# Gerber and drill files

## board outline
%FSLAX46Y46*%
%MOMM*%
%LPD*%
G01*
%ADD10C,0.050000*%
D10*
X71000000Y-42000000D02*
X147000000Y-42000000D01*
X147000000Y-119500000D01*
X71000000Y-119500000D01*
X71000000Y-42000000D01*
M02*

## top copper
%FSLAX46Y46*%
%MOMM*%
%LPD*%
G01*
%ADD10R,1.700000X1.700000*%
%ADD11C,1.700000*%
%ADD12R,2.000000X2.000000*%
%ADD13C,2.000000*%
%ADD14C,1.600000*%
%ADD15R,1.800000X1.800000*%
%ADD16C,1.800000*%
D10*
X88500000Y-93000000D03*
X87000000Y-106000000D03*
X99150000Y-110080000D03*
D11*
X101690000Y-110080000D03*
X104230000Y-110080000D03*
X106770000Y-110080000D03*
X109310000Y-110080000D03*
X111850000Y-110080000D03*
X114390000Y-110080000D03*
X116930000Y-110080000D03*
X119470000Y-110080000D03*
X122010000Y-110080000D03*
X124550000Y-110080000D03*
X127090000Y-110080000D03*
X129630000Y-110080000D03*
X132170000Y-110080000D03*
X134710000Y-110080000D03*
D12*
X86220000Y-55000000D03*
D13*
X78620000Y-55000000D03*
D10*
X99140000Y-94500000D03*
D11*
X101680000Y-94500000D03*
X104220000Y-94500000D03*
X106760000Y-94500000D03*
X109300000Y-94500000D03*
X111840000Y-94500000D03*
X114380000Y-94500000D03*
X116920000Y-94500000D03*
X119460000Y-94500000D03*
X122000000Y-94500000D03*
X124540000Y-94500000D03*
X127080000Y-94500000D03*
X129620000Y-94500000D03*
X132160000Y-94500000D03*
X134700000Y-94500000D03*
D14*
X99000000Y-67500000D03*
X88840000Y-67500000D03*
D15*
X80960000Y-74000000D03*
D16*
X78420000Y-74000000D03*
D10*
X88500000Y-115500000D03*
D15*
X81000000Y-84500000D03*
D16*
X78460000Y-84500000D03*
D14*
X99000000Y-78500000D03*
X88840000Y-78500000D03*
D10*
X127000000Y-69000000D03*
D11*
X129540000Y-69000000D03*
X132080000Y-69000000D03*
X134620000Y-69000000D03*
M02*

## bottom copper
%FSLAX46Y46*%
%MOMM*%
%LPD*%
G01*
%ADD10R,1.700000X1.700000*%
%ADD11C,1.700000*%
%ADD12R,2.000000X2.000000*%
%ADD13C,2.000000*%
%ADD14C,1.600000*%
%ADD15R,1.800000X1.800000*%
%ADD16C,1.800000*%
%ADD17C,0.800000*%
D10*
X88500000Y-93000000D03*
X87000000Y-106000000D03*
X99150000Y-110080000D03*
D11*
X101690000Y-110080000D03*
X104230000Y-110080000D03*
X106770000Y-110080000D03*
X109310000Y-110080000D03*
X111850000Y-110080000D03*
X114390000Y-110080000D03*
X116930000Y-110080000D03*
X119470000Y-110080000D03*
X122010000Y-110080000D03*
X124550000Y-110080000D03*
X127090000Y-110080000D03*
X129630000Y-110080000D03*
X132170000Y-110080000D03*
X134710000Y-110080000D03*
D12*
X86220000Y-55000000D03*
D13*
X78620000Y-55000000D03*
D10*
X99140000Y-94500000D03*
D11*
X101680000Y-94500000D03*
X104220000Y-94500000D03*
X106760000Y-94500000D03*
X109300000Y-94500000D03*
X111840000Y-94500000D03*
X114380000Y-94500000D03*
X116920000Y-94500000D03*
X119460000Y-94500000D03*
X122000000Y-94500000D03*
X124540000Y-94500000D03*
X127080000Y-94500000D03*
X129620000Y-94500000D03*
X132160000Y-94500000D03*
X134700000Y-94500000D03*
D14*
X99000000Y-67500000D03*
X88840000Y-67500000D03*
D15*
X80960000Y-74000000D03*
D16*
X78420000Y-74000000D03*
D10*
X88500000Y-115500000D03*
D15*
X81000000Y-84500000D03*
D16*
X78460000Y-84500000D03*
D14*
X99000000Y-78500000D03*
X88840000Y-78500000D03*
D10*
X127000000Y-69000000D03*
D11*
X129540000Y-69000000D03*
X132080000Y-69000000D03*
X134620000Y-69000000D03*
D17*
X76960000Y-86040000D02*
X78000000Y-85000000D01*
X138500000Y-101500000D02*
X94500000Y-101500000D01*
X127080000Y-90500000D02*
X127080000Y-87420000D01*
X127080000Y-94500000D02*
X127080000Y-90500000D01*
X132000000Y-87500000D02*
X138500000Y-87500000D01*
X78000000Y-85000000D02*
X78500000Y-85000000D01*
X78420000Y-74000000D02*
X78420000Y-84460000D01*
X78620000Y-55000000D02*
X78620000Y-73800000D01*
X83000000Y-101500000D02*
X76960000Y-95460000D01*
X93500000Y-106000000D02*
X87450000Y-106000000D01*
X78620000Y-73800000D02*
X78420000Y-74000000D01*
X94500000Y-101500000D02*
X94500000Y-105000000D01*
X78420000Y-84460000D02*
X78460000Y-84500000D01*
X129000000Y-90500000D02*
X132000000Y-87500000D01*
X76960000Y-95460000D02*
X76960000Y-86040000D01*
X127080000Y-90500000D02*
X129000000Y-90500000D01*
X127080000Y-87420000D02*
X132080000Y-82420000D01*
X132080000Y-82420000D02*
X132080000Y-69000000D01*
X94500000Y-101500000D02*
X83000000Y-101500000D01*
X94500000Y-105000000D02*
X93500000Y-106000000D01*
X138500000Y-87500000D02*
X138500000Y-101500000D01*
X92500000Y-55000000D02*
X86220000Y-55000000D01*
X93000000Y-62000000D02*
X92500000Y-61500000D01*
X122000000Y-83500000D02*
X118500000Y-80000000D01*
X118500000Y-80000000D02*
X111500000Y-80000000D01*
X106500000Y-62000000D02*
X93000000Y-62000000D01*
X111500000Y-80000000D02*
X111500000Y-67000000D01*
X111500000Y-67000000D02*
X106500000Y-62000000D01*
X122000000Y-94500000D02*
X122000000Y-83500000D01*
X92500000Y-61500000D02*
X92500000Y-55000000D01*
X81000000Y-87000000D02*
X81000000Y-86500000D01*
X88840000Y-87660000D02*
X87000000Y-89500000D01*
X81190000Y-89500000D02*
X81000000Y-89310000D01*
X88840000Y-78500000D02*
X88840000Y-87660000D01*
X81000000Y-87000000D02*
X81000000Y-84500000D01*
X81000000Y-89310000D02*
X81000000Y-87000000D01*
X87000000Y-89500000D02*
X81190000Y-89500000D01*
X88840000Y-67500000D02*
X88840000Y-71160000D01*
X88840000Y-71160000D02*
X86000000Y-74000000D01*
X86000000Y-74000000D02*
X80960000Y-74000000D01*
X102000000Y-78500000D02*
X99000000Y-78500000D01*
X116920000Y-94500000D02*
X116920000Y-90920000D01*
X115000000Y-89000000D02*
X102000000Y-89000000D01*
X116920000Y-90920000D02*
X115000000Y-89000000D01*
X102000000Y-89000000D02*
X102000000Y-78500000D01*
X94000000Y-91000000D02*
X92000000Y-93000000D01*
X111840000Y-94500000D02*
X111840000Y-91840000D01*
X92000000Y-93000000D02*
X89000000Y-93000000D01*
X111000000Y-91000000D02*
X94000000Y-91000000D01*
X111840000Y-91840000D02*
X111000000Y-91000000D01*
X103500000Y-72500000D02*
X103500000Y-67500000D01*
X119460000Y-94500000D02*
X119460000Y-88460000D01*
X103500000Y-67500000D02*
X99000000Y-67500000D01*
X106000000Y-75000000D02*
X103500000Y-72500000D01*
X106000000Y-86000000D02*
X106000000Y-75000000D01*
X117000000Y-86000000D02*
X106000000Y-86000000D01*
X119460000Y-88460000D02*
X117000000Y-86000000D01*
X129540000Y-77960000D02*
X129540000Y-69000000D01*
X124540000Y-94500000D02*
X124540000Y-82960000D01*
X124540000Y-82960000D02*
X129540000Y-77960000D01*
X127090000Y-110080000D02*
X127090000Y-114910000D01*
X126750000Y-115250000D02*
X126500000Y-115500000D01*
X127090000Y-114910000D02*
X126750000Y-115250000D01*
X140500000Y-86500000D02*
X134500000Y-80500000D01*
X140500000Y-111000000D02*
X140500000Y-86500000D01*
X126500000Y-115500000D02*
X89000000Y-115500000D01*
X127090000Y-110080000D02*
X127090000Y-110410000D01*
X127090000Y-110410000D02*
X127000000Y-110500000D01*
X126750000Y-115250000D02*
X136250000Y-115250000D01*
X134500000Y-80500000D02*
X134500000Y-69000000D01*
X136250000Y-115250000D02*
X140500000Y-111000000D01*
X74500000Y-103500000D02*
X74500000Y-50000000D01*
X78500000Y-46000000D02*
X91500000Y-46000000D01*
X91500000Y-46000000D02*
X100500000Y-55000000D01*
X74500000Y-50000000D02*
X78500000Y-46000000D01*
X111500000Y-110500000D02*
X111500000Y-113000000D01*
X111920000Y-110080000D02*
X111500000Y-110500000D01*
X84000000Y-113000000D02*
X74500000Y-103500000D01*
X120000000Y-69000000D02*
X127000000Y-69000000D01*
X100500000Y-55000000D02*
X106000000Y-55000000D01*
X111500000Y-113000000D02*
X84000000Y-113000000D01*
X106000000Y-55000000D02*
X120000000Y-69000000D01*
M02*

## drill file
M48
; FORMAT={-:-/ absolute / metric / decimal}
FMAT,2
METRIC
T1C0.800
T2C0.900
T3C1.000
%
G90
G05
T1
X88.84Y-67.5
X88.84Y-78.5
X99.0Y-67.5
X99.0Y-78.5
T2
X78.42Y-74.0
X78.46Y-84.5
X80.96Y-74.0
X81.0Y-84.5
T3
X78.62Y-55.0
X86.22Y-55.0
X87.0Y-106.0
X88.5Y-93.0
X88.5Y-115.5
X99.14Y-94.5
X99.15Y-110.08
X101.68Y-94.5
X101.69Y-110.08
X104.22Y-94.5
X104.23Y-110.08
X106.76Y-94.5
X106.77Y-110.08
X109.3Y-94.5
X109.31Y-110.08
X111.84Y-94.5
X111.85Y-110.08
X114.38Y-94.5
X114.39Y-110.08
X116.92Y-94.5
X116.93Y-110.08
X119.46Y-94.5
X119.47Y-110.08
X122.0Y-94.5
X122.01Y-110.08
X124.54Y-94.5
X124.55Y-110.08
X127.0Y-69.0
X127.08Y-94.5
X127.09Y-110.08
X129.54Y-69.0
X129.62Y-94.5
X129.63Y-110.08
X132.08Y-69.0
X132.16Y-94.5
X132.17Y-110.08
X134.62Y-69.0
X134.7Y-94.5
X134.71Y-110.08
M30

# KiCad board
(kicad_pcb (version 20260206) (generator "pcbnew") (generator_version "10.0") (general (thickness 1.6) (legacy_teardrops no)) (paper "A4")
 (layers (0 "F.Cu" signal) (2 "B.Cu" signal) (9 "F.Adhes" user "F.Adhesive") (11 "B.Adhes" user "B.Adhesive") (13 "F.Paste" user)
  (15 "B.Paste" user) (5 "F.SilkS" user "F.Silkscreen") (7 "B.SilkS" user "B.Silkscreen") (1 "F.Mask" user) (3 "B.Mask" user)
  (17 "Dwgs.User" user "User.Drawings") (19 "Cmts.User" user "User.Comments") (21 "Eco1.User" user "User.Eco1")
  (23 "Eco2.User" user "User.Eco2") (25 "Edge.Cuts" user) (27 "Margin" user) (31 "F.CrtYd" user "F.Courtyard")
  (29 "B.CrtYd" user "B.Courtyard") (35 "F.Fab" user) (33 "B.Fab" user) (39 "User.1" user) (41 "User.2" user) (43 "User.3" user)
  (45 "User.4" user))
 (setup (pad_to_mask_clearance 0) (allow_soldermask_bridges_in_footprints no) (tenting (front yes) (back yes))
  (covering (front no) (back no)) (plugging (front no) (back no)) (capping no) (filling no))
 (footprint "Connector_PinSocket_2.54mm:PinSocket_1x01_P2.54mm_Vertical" (layer "F.Cu") (at 88.5 93 90)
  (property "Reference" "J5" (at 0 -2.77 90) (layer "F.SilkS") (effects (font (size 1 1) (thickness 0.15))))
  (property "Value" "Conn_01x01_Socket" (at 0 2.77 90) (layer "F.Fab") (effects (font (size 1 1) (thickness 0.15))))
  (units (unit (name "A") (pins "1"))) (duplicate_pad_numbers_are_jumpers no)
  (pad "1" thru_hole rect (at 0 0 90) (size 1.7 1.7) (drill 1) (layers "*.Cu" "*.Mask") (remove_unused_layers no) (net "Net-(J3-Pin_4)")))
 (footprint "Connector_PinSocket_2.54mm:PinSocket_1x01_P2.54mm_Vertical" (layer "F.Cu") (at 87 106 90)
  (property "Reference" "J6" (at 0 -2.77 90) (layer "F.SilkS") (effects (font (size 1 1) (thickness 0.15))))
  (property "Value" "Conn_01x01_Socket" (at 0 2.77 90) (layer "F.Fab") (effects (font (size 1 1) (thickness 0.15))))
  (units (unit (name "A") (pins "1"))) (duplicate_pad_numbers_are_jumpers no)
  (pad "1" thru_hole rect (at 0 0 90) (size 1.7 1.7) (drill 1) (layers "*.Cu" "*.Mask") (remove_unused_layers no) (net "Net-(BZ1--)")))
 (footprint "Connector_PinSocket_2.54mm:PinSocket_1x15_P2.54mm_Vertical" (layer "F.Cu") (at 99.15 110.08 90)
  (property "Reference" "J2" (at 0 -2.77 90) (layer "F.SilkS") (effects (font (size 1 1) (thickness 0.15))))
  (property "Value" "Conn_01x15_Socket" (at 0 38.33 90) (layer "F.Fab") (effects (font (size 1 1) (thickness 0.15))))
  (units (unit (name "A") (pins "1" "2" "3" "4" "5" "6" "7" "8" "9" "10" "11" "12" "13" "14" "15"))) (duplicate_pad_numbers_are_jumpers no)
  (pad "1" thru_hole rect (at 0 0 90) (size 1.7 1.7) (drill 1) (layers "*.Cu" "*.Mask") (remove_unused_layers no)
   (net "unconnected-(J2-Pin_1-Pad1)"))
  (pad "2" thru_hole circle (at 0 2.54 90) (size 1.7 1.7) (drill 1) (layers "*.Cu" "*.Mask") (remove_unused_layers no)
   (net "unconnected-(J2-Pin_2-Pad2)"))
  (pad "3" thru_hole circle (at 0 5.08 90) (size 1.7 1.7) (drill 1) (layers "*.Cu" "*.Mask") (remove_unused_layers no)
   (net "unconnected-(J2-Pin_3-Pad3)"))
  (pad "4" thru_hole circle (at 0 7.62 90) (size 1.7 1.7) (drill 1) (layers "*.Cu" "*.Mask") (remove_unused_layers no)
   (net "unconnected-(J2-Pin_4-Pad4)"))
  (pad "5" thru_hole circle (at 0 10.16 90) (size 1.7 1.7) (drill 1) (layers "*.Cu" "*.Mask") (remove_unused_layers no)
   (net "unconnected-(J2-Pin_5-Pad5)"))
  (pad "6" thru_hole circle (at 0 12.7 90) (size 1.7 1.7) (drill 1) (layers "*.Cu" "*.Mask") (remove_unused_layers no)
   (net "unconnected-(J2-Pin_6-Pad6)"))
  (pad "7" thru_hole circle (at 0 15.24 90) (size 1.7 1.7) (drill 1) (layers "*.Cu" "*.Mask") (remove_unused_layers no)
   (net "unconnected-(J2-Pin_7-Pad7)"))
  (pad "8" thru_hole circle (at 0 17.78 90) (size 1.7 1.7) (drill 1) (layers "*.Cu" "*.Mask") (remove_unused_layers no)
   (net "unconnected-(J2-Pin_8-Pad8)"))
  (pad "9" thru_hole circle (at 0 20.32 90) (size 1.7 1.7) (drill 1) (layers "*.Cu" "*.Mask") (remove_unused_layers no)
   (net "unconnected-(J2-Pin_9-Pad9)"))
  (pad "10" thru_hole circle (at 0 22.86 90) (size 1.7 1.7) (drill 1) (layers "*.Cu" "*.Mask") (remove_unused_layers no)
   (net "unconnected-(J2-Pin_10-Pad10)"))
  (pad "11" thru_hole circle (at 0 25.4 90) (size 1.7 1.7) (drill 1) (layers "*.Cu" "*.Mask") (remove_unused_layers no)
   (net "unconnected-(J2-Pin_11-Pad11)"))
  (pad "12" thru_hole circle (at 0 27.94 90) (size 1.7 1.7) (drill 1) (layers "*.Cu" "*.Mask") (remove_unused_layers no)
   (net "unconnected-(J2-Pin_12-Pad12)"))
  (pad "13" thru_hole circle (at 0 30.48 90) (size 1.7 1.7) (drill 1) (layers "*.Cu" "*.Mask") (remove_unused_layers no)
   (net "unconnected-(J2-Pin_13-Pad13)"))
  (pad "14" thru_hole circle (at 0 33.02 90) (size 1.7 1.7) (drill 1) (layers "*.Cu" "*.Mask") (remove_unused_layers no)
   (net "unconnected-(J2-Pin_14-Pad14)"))
  (pad "15" thru_hole circle (at 0 35.56 90) (size 1.7 1.7) (drill 1) (layers "*.Cu" "*.Mask") (remove_unused_layers no)
   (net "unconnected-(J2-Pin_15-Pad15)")))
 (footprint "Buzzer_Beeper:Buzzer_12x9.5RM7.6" (layer "F.Cu") (at 86.22 55 180)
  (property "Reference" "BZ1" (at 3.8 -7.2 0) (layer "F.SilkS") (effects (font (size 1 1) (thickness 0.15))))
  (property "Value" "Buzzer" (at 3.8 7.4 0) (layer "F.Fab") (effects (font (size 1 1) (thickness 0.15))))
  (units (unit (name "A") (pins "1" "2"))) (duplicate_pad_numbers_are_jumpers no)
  (pad "1" thru_hole rect (at 0 0 180) (size 2 2) (drill 1) (layers "*.Cu" "*.Mask") (remove_unused_layers no) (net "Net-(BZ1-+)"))
  (pad "2" thru_hole circle (at 7.6 0 180) (size 2 2) (drill 1) (layers "*.Cu" "*.Mask") (remove_unused_layers no) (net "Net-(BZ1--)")))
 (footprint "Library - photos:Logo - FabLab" (layer "F.Cu") (at 115.5 49)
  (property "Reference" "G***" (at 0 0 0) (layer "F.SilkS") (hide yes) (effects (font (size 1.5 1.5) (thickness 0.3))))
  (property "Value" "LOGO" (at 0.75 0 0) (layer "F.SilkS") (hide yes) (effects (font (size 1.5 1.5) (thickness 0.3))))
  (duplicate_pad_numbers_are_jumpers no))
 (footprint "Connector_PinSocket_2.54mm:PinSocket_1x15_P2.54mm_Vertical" (layer "F.Cu") (at 99.14 94.5 90)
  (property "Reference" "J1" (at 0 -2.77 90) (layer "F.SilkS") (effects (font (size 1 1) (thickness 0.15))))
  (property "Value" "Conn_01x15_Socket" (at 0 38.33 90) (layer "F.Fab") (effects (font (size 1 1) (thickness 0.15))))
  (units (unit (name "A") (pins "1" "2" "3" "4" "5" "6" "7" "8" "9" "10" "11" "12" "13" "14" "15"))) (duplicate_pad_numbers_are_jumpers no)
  (pad "1" thru_hole rect (at 0 0 90) (size 1.7 1.7) (drill 1) (layers "*.Cu" "*.Mask") (remove_unused_layers no)
   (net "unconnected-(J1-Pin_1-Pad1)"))
  (pad "2" thru_hole circle (at 0 2.54 90) (size 1.7 1.7) (drill 1) (layers "*.Cu" "*.Mask") (remove_unused_layers no)
   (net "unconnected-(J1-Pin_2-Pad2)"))
  (pad "3" thru_hole circle (at 0 5.08 90) (size 1.7 1.7) (drill 1) (layers "*.Cu" "*.Mask") (remove_unused_layers no)
   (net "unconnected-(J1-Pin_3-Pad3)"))
  (pad "4" thru_hole circle (at 0 7.62 90) (size 1.7 1.7) (drill 1) (layers "*.Cu" "*.Mask") (remove_unused_layers no)
   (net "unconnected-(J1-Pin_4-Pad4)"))
  (pad "5" thru_hole circle (at 0 10.16 90) (size 1.7 1.7) (drill 1) (layers "*.Cu" "*.Mask") (remove_unused_layers no)
   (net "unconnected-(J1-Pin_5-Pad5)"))
  (pad "6" thru_hole circle (at 0 12.7 90) (size 1.7 1.7) (drill 1) (layers "*.Cu" "*.Mask") (remove_unused_layers no)
   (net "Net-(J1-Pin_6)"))
  (pad "7" thru_hole circle (at 0 15.24 90) (size 1.7 1.7) (drill 1) (layers "*.Cu" "*.Mask") (remove_unused_layers no)
   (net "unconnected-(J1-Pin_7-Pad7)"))
  (pad "8" thru_hole circle (at 0 17.78 90) (size 1.7 1.7) (drill 1) (layers "*.Cu" "*.Mask") (remove_unused_layers no)
   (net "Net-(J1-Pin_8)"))
  (pad "9" thru_hole circle (at 0 20.32 90) (size 1.7 1.7) (drill 1) (layers "*.Cu" "*.Mask") (remove_unused_layers no)
   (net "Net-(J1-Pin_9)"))
  (pad "10" thru_hole circle (at 0 22.86 90) (size 1.7 1.7) (drill 1) (layers "*.Cu" "*.Mask") (remove_unused_layers no) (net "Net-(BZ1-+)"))
  (pad "11" thru_hole circle (at 0 25.4 90) (size 1.7 1.7) (drill 1) (layers "*.Cu" "*.Mask") (remove_unused_layers no)
   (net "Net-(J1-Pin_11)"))
  (pad "12" thru_hole circle (at 0 27.94 90) (size 1.7 1.7) (drill 1) (layers "*.Cu" "*.Mask") (remove_unused_layers no) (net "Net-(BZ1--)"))
  (pad "13" thru_hole circle (at 0 30.48 90) (size 1.7 1.7) (drill 1) (layers "*.Cu" "*.Mask") (remove_unused_layers no)
   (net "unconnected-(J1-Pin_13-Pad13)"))
  (pad "14" thru_hole circle (at 0 33.02 90) (size 1.7 1.7) (drill 1) (layers "*.Cu" "*.Mask") (remove_unused_layers no)
   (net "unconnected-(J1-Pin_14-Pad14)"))
  (pad "15" thru_hole circle (at 0 35.56 90) (size 1.7 1.7) (drill 1) (layers "*.Cu" "*.Mask") (remove_unused_layers no)
   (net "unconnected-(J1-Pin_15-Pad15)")))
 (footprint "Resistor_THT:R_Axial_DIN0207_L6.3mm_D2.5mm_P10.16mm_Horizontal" (layer "F.Cu") (at 99 67.5 180)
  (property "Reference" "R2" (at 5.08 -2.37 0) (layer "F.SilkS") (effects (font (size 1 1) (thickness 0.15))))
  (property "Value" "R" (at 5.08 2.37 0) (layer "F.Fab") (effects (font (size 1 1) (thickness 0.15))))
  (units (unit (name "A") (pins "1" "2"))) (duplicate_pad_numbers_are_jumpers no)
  (pad "1" thru_hole circle (at 0 0 180) (size 1.6 1.6) (drill 0.8) (layers "*.Cu" "*.Mask") (remove_unused_layers no)
   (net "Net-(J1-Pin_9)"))
  (pad "2" thru_hole circle (at 10.16 0 180) (size 1.6 1.6) (drill 0.8) (layers "*.Cu" "*.Mask") (remove_unused_layers no)
   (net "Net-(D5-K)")))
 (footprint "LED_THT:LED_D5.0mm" (layer "F.Cu") (at 80.96 74 180)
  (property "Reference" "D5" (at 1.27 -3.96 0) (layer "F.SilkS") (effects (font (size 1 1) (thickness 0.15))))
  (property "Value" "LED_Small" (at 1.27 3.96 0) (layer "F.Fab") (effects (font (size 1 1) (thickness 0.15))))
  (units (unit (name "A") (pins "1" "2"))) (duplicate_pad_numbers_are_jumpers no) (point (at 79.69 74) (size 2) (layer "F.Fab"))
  (pad "1" thru_hole rect (at 0 0 180) (size 1.8 1.8) (drill 0.9) (layers "*.Cu" "*.Mask") (remove_unused_layers no) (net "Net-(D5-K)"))
  (pad "2" thru_hole circle (at 2.54 0 180) (size 1.8 1.8) (drill 0.9) (layers "*.Cu" "*.Mask") (remove_unused_layers no)
   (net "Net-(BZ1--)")))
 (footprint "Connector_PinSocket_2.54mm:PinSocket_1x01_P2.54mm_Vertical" (layer "F.Cu") (at 88.5 115.5 90)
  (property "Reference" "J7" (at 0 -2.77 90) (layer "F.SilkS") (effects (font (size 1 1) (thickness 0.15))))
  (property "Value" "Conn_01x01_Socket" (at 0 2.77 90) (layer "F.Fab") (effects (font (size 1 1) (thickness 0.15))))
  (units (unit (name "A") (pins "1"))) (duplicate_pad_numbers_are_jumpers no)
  (pad "1" thru_hole rect (at 0 0 90) (size 1.7 1.7) (drill 1) (layers "*.Cu" "*.Mask") (remove_unused_layers no) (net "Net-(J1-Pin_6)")))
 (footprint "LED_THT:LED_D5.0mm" (layer "F.Cu") (at 81 84.5 180)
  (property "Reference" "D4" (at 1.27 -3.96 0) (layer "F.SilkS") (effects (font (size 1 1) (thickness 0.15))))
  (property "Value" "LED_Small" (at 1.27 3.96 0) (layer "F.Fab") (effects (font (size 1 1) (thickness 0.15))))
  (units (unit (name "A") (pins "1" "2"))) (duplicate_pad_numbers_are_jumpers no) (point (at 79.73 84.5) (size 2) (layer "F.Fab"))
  (pad "1" thru_hole rect (at 0 0 180) (size 1.8 1.8) (drill 0.9) (layers "*.Cu" "*.Mask") (remove_unused_layers no) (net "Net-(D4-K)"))
  (pad "2" thru_hole circle (at 2.54 0 180) (size 1.8 1.8) (drill 0.9) (layers "*.Cu" "*.Mask") (remove_unused_layers no)
   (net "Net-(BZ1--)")))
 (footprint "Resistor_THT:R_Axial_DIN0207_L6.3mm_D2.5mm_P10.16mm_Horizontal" (layer "F.Cu") (at 99 78.5 180)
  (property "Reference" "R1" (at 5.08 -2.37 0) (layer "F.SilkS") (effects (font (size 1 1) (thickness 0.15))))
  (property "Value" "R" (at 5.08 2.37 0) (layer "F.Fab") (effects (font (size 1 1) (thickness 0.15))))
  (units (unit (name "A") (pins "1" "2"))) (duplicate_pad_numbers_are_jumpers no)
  (pad "1" thru_hole circle (at 0 0 180) (size 1.6 1.6) (drill 0.8) (layers "*.Cu" "*.Mask") (remove_unused_layers no)
   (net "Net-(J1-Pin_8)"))
  (pad "2" thru_hole circle (at 10.16 0 180) (size 1.6 1.6) (drill 0.8) (layers "*.Cu" "*.Mask") (remove_unused_layers no)
   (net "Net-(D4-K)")))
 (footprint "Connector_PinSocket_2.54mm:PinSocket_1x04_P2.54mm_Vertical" (layer "F.Cu") (at 127 69 90)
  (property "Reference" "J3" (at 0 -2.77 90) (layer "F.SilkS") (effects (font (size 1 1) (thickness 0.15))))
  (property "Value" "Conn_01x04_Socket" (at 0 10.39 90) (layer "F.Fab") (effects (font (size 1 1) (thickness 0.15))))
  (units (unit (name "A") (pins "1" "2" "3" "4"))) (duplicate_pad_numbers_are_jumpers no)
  (pad "1" thru_hole rect (at 0 0 90) (size 1.7 1.7) (drill 1) (layers "*.Cu" "*.Mask") (remove_unused_layers no)
   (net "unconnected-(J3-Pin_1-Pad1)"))
  (pad "2" thru_hole circle (at 0 2.54 90) (size 1.7 1.7) (drill 1) (layers "*.Cu" "*.Mask") (remove_unused_layers no)
   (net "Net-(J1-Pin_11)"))
  (pad "3" thru_hole circle (at 0 5.08 90) (size 1.7 1.7) (drill 1) (layers "*.Cu" "*.Mask") (remove_unused_layers no) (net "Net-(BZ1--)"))
  (pad "4" thru_hole circle (at 0 7.62 90) (size 1.7 1.7) (drill 1) (layers "*.Cu" "*.Mask") (remove_unused_layers no)
   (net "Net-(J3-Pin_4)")))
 (gr_rect (start 71 42) (end 147 119.5) (stroke (width 0.05) (type default)) (fill no) (layer "Edge.Cuts"))
 (segment (start 76.96 86.04) (end 78 85) (width 0.8) (layer "B.Cu") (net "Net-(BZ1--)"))
 (segment (start 138.5 101.5) (end 94.5 101.5) (width 0.8) (layer "B.Cu") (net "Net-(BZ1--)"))
 (segment (start 127.08 90.5) (end 127.08 87.42) (width 0.8) (layer "B.Cu") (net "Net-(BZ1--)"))
 (segment (start 127.08 94.5) (end 127.08 90.5) (width 0.8) (layer "B.Cu") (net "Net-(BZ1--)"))
 (segment (start 132 87.5) (end 138.5 87.5) (width 0.8) (layer "B.Cu") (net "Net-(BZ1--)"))
 (segment (start 78 85) (end 78.5 85) (width 0.8) (layer "B.Cu") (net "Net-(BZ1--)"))
 (segment (start 78.42 74) (end 78.42 84.46) (width 0.8) (layer "B.Cu") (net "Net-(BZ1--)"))
 (segment (start 78.62 55) (end 78.62 73.8) (width 0.8) (layer "B.Cu") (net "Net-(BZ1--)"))
 (segment (start 83 101.5) (end 76.96 95.46) (width 0.8) (layer "B.Cu") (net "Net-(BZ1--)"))
 (segment (start 93.5 106) (end 87.45 106) (width 0.8) (layer "B.Cu") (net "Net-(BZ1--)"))
 (segment (start 78.62 73.8) (end 78.42 74) (width 0.8) (layer "B.Cu") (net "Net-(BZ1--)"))
 (segment (start 94.5 101.5) (end 94.5 105) (width 0.8) (layer "B.Cu") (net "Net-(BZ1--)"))
 (segment (start 78.42 84.46) (end 78.46 84.5) (width 0.8) (layer "B.Cu") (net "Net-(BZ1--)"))
 (segment (start 129 90.5) (end 132 87.5) (width 0.8) (layer "B.Cu") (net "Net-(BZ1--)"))
 (segment (start 76.96 95.46) (end 76.96 86.04) (width 0.8) (layer "B.Cu") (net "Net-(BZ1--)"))
 (segment (start 127.08 90.5) (end 129 90.5) (width 0.8) (layer "B.Cu") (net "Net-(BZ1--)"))
 (segment (start 127.08 87.42) (end 132.08 82.42) (width 0.8) (layer "B.Cu") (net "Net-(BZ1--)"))
 (segment (start 132.08 82.42) (end 132.08 69) (width 0.8) (layer "B.Cu") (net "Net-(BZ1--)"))
 (segment (start 94.5 101.5) (end 83 101.5) (width 0.8) (layer "B.Cu") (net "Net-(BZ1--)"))
 (segment (start 94.5 105) (end 93.5 106) (width 0.8) (layer "B.Cu") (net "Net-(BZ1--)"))
 (segment (start 138.5 87.5) (end 138.5 101.5) (width 0.8) (layer "B.Cu") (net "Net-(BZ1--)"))
 (segment (start 92.5 55) (end 86.22 55) (width 0.8) (layer "B.Cu") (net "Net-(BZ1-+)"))
 (segment (start 93 62) (end 92.5 61.5) (width 0.8) (layer "B.Cu") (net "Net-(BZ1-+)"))
 (segment (start 122 83.5) (end 118.5 80) (width 0.8) (layer "B.Cu") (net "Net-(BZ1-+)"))
 (segment (start 118.5 80) (end 111.5 80) (width 0.8) (layer "B.Cu") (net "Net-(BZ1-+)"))
 (segment (start 106.5 62) (end 93 62) (width 0.8) (layer "B.Cu") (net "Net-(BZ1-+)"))
 (segment (start 111.5 80) (end 111.5 67) (width 0.8) (layer "B.Cu") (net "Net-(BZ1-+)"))
 (segment (start 111.5 67) (end 106.5 62) (width 0.8) (layer "B.Cu") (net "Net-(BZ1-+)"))
 (segment (start 122 94.5) (end 122 83.5) (width 0.8) (layer "B.Cu") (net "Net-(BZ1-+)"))
 (segment (start 92.5 61.5) (end 92.5 55) (width 0.8) (layer "B.Cu") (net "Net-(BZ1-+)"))
 (segment (start 81 87) (end 81 86.5) (width 0.8) (layer "B.Cu") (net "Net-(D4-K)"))
 (segment (start 88.84 87.66) (end 87 89.5) (width 0.8) (layer "B.Cu") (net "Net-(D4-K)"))
 (segment (start 81.19 89.5) (end 81 89.31) (width 0.8) (layer "B.Cu") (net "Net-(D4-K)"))
 (segment (start 88.84 78.5) (end 88.84 87.66) (width 0.8) (layer "B.Cu") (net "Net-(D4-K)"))
 (segment (start 81 87) (end 81 84.5) (width 0.8) (layer "B.Cu") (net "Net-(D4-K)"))
 (segment (start 81 89.31) (end 81 87) (width 0.8) (layer "B.Cu") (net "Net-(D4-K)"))
 (segment (start 87 89.5) (end 81.19 89.5) (width 0.8) (layer "B.Cu") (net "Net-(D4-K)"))
 (segment (start 88.84 67.5) (end 88.84 71.16) (width 0.8) (layer "B.Cu") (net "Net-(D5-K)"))
 (segment (start 88.84 71.16) (end 86 74) (width 0.8) (layer "B.Cu") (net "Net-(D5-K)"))
 (segment (start 86 74) (end 80.96 74) (width 0.8) (layer "B.Cu") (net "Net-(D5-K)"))
 (segment (start 102 78.5) (end 99 78.5) (width 0.8) (layer "B.Cu") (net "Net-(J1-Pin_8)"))
 (segment (start 116.92 94.5) (end 116.92 90.92) (width 0.8) (layer "B.Cu") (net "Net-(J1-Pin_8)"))
 (segment (start 115 89) (end 102 89) (width 0.8) (layer "B.Cu") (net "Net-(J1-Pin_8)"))
 (segment (start 116.92 90.92) (end 115 89) (width 0.8) (layer "B.Cu") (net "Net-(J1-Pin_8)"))
 (segment (start 102 89) (end 102 78.5) (width 0.8) (layer "B.Cu") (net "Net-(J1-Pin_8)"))
 (segment (start 94 91) (end 92 93) (width 0.8) (layer "B.Cu") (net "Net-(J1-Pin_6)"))
 (segment (start 111.84 94.5) (end 111.84 91.84) (width 0.8) (layer "B.Cu") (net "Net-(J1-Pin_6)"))
 (segment (start 92 93) (end 89 93) (width 0.8) (layer "B.Cu") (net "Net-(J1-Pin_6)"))
 (segment (start 111 91) (end 94 91) (width 0.8) (layer "B.Cu") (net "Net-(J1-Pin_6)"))
 (segment (start 111.84 91.84) (end 111 91) (width 0.8) (layer "B.Cu") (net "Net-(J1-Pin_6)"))
 (segment (start 103.5 72.5) (end 103.5 67.5) (width 0.8) (layer "B.Cu") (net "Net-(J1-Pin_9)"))
 (segment (start 119.46 94.5) (end 119.46 88.46) (width 0.8) (layer "B.Cu") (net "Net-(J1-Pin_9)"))
 (segment (start 103.5 67.5) (end 99 67.5) (width 0.8) (layer "B.Cu") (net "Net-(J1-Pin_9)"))
 (segment (start 106 75) (end 103.5 72.5) (width 0.8) (layer "B.Cu") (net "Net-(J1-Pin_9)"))
 (segment (start 106 86) (end 106 75) (width 0.8) (layer "B.Cu") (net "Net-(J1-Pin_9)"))
 (segment (start 117 86) (end 106 86) (width 0.8) (layer "B.Cu") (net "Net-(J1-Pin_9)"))
 (segment (start 119.46 88.46) (end 117 86) (width 0.8) (layer "B.Cu") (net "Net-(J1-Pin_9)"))
 (segment (start 129.54 77.96) (end 129.54 69) (width 0.8) (layer "B.Cu") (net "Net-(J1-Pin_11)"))
 (segment (start 124.54 94.5) (end 124.54 82.96) (width 0.8) (layer "B.Cu") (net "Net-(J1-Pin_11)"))
 (segment (start 124.54 82.96) (end 129.54 77.96) (width 0.8) (layer "B.Cu") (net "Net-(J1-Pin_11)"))
 (segment (start 127.09 110.08) (end 127.09 114.91) (width 0.8) (layer "B.Cu") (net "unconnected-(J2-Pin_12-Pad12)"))
 (segment (start 126.75 115.25) (end 126.5 115.5) (width 0.8) (layer "B.Cu") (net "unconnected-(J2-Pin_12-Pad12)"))
 (segment (start 127.09 114.91) (end 126.75 115.25) (width 0.8) (layer "B.Cu") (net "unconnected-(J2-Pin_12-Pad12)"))
 (segment (start 140.5 86.5) (end 134.5 80.5) (width 0.8) (layer "B.Cu") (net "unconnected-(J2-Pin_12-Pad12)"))
 (segment (start 140.5 111) (end 140.5 86.5) (width 0.8) (layer "B.Cu") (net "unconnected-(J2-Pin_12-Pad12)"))
 (segment (start 126.5 115.5) (end 89 115.5) (width 0.8) (layer "B.Cu") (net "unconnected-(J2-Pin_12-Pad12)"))
 (segment (start 127.09 110.08) (end 127.09 110.41) (width 0.8) (layer "B.Cu") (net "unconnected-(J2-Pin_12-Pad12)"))
 (segment (start 127.09 110.41) (end 127 110.5) (width 0.8) (layer "B.Cu") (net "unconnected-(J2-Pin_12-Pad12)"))
 (segment (start 126.75 115.25) (end 136.25 115.25) (width 0.8) (layer "B.Cu") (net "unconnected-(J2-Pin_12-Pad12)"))
 (segment (start 134.5 80.5) (end 134.5 69) (width 0.8) (layer "B.Cu") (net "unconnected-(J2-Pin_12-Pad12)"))
 (segment (start 136.25 115.25) (end 140.5 111) (width 0.8) (layer "B.Cu") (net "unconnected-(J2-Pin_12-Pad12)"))
 (segment (start 74.5 103.5) (end 74.5 50) (width 0.8) (layer "B.Cu") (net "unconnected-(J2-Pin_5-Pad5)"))
 (segment (start 78.5 46) (end 91.5 46) (width 0.8) (layer "B.Cu") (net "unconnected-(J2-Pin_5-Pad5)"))
 (segment (start 91.5 46) (end 100.5 55) (width 0.8) (layer "B.Cu") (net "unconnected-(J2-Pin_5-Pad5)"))
 (segment (start 74.5 50) (end 78.5 46) (width 0.8) (layer "B.Cu") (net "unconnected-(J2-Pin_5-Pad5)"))
 (segment (start 111.5 110.5) (end 111.5 113) (width 0.8) (layer "B.Cu") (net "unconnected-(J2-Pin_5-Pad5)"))
 (segment (start 111.92 110.08) (end 111.5 110.5) (width 0.8) (layer "B.Cu") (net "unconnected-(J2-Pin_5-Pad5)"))
 (segment (start 84 113) (end 74.5 103.5) (width 0.8) (layer "B.Cu") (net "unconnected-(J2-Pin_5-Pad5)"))
 (segment (start 120 69) (end 127 69) (width 0.8) (layer "B.Cu") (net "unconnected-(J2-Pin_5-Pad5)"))
 (segment (start 100.5 55) (end 106 55) (width 0.8) (layer "B.Cu") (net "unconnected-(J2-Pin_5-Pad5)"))
 (segment (start 111.5 113) (end 84 113) (width 0.8) (layer "B.Cu") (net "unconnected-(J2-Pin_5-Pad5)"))
 (segment (start 106 55) (end 120 69) (width 0.8) (layer "B.Cu") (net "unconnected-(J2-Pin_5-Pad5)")))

